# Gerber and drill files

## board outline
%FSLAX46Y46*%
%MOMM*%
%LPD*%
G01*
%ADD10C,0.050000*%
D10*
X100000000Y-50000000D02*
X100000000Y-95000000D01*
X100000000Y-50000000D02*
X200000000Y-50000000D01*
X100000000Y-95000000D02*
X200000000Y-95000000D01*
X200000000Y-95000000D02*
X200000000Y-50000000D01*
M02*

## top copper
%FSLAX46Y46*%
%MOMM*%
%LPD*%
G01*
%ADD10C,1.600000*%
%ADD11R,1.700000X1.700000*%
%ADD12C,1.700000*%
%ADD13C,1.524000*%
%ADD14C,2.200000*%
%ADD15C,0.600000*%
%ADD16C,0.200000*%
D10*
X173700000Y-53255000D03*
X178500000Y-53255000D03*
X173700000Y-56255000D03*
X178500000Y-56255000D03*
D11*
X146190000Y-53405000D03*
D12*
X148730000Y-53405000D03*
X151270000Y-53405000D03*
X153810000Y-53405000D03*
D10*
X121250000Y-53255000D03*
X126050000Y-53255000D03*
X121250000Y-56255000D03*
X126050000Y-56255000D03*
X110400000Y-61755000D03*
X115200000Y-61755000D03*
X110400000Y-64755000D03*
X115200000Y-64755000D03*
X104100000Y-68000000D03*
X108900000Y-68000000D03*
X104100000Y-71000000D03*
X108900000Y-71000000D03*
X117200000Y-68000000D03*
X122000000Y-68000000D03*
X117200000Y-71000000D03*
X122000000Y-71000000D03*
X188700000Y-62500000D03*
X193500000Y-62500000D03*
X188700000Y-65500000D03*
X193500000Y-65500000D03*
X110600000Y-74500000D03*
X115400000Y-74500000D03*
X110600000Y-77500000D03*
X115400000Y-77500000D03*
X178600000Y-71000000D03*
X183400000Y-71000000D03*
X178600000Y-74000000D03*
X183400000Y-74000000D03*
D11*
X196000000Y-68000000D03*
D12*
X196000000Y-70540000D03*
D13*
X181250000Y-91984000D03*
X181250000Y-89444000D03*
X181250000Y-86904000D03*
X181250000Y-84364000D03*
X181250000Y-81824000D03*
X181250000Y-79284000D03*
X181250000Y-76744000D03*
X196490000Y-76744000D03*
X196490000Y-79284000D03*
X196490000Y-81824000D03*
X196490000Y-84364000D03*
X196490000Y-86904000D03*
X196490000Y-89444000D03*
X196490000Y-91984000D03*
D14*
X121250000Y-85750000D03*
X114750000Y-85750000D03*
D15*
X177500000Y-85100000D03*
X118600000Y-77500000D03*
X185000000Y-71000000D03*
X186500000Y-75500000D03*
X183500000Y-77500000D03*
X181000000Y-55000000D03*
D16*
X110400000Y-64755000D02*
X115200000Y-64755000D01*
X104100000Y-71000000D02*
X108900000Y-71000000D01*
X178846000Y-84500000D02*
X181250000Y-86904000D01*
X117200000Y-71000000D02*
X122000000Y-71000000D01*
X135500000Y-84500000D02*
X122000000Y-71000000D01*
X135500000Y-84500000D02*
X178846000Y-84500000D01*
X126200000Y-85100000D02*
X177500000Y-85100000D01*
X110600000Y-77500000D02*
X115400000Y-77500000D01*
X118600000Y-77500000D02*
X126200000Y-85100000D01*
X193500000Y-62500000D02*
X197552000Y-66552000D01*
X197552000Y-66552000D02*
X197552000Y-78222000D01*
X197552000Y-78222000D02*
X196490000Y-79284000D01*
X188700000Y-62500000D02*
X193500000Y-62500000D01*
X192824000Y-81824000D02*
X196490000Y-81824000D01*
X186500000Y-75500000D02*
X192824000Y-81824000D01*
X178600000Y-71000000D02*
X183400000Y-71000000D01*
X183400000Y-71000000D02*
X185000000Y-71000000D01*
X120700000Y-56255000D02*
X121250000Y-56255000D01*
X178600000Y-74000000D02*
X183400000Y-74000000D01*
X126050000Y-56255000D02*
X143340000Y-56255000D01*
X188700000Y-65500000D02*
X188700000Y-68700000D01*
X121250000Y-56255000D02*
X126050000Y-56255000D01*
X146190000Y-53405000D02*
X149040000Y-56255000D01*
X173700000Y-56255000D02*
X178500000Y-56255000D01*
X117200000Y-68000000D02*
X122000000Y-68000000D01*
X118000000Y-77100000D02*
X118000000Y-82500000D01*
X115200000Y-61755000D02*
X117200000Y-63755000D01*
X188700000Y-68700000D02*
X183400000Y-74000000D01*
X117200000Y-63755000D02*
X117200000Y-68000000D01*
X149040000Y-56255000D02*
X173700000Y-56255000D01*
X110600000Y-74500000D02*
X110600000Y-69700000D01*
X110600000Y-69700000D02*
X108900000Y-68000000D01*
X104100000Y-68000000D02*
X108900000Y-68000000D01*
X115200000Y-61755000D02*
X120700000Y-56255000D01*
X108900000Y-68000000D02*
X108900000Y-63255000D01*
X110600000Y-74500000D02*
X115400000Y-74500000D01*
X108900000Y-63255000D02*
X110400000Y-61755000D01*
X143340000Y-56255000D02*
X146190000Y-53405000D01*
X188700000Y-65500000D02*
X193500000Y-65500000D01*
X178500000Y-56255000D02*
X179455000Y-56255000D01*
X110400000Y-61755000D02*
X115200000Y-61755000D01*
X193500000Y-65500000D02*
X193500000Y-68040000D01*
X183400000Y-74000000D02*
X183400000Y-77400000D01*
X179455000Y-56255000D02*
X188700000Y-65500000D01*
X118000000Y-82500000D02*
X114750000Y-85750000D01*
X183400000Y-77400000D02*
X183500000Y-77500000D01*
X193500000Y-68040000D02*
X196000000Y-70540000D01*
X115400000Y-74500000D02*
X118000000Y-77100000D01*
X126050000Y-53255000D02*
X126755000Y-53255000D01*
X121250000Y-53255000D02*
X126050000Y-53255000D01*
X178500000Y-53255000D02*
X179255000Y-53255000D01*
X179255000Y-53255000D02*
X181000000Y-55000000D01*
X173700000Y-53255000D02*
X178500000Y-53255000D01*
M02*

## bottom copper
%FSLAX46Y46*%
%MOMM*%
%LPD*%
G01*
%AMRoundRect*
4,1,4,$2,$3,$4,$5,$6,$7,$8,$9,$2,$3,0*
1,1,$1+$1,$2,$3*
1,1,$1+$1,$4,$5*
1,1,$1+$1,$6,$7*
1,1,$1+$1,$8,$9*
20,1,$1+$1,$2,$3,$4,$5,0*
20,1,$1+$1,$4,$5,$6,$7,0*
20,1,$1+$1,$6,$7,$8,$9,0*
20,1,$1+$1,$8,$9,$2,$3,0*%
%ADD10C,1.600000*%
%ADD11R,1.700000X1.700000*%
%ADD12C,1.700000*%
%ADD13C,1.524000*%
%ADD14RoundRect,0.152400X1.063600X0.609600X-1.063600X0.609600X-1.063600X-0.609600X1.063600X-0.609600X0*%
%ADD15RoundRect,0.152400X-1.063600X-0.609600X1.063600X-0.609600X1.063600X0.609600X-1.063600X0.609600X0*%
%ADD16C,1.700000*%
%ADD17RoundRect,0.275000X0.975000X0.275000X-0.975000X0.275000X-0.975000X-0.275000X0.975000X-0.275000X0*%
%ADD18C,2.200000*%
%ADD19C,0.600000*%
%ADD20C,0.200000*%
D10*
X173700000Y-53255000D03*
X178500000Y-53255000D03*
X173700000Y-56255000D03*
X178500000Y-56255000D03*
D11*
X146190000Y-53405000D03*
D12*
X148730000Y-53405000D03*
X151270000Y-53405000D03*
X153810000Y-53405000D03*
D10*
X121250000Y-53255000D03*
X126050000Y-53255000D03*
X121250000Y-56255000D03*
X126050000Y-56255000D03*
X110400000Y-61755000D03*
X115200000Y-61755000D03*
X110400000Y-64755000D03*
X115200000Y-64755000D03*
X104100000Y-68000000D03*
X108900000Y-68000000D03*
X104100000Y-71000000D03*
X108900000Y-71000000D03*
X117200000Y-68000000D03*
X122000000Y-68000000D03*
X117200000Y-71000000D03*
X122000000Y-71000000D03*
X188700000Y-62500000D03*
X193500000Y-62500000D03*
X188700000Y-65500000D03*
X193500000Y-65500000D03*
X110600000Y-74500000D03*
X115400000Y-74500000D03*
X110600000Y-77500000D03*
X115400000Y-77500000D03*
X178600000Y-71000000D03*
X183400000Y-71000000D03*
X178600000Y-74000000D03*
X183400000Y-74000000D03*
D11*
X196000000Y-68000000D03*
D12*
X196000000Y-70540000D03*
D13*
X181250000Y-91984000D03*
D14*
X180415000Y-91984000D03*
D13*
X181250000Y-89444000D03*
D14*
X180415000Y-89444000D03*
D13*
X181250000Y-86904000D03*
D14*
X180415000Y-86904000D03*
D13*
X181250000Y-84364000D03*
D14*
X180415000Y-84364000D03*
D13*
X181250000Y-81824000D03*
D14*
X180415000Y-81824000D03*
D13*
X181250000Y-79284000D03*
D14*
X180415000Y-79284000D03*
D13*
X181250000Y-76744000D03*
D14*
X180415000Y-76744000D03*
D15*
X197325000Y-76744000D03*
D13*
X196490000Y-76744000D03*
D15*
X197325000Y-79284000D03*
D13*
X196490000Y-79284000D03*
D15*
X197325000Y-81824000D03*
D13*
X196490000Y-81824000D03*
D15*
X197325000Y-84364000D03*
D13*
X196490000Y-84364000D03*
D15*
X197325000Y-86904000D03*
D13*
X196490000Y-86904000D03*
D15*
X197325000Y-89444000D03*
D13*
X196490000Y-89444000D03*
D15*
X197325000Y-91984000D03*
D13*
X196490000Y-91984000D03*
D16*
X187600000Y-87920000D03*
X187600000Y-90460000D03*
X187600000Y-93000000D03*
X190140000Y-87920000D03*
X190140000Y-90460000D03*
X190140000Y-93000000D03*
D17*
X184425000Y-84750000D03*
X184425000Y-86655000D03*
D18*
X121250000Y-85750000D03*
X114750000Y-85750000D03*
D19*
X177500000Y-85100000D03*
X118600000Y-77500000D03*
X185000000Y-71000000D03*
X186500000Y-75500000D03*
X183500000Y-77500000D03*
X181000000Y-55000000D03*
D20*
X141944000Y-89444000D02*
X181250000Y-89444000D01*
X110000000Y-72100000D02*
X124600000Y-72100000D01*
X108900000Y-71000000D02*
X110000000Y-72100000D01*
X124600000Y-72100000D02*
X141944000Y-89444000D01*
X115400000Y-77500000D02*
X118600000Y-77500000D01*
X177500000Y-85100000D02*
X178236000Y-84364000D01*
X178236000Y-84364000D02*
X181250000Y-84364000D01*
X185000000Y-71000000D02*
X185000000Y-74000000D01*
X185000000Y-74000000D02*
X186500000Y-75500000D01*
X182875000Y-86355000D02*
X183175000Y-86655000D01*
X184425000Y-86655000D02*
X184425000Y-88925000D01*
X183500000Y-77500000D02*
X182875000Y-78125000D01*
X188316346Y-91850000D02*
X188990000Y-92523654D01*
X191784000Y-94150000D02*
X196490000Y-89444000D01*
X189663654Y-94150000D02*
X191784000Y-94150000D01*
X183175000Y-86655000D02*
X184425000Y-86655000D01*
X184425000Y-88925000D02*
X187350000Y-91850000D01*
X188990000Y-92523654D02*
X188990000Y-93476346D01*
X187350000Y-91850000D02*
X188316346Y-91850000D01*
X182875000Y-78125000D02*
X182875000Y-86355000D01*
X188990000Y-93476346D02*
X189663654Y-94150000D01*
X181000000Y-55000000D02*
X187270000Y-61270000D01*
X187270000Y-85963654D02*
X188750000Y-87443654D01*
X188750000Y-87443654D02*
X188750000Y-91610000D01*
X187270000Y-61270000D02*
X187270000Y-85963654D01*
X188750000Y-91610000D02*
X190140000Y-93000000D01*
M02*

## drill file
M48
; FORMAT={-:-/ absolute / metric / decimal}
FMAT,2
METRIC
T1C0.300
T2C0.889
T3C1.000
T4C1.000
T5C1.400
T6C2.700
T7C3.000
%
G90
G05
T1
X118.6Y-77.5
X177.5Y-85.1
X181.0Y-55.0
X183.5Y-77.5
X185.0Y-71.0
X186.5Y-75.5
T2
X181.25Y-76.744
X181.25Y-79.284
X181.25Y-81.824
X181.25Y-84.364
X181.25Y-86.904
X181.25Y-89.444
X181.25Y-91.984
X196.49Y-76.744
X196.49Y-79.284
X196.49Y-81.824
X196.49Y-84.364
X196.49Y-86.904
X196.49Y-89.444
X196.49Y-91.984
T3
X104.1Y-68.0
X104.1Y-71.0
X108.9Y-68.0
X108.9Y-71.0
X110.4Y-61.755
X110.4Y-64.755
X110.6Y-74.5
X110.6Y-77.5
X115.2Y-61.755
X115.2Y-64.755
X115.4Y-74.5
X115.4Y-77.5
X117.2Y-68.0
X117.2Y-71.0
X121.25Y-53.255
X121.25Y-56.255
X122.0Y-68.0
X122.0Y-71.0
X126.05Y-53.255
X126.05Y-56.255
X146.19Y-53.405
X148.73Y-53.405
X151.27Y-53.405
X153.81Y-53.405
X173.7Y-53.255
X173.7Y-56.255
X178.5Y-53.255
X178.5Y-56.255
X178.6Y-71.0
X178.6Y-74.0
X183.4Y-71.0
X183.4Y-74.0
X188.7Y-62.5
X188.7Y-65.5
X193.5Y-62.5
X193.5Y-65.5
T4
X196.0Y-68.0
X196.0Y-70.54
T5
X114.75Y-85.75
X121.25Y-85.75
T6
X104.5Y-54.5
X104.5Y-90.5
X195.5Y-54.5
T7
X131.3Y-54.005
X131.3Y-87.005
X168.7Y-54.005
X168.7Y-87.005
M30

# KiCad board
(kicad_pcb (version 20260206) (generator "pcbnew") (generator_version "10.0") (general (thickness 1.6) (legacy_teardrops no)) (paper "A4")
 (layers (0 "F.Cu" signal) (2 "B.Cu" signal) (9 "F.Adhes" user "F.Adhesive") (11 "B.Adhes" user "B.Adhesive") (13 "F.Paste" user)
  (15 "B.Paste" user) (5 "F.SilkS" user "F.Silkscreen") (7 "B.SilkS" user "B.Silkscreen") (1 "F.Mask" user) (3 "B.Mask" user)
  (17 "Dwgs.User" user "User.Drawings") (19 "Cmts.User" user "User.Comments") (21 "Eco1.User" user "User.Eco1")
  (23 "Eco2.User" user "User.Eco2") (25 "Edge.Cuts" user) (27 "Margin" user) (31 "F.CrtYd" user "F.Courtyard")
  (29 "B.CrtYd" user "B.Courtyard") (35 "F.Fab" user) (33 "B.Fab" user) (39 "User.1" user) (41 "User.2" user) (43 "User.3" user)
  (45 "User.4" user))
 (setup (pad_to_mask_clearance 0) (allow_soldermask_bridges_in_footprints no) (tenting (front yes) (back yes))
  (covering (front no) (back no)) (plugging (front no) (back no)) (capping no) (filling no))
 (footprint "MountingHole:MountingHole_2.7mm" (layer "F.Cu") (at 104.5 90.5)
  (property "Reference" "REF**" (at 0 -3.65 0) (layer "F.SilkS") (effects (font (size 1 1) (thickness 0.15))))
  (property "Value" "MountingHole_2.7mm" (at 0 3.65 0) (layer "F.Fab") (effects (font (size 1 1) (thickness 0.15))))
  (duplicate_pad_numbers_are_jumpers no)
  (pad "" np_thru_hole circle (at 0 0) (size 2.7 2.7) (drill 2.7) (layers "*.Cu" "*.Mask")))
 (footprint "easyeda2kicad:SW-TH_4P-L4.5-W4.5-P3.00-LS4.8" (layer "F.Cu") (at 176.1 54.755)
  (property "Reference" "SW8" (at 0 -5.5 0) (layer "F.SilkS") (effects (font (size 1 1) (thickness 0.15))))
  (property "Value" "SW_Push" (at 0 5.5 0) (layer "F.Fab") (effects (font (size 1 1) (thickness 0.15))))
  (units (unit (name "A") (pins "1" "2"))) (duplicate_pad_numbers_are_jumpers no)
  (pad "1" thru_hole circle (at -2.4 -1.5) (size 1.6 1.6) (drill 0.999998) (layers "*.Cu" "*.Mask") (remove_unused_layers no)
   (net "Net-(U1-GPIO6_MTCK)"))
  (pad "1" thru_hole circle (at 2.4 -1.5) (size 1.6 1.6) (drill 0.999998) (layers "*.Cu" "*.Mask") (remove_unused_layers no)
   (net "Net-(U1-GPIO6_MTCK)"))
  (pad "2" thru_hole circle (at -2.4 1.5) (size 1.6 1.6) (drill 0.999998) (layers "*.Cu" "*.Mask") (remove_unused_layers no) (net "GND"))
  (pad "2" thru_hole circle (at 2.4 1.5) (size 1.6 1.6) (drill 0.999998) (layers "*.Cu" "*.Mask") (remove_unused_layers no) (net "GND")))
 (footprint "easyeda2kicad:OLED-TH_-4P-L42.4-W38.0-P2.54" (layer "F.Cu") (at 150 53.405)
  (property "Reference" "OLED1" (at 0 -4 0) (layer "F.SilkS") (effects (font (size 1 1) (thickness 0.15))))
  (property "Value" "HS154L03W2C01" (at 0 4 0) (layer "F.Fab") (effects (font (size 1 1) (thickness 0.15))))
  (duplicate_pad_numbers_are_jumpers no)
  (pad "" np_thru_hole circle (at -18.7 0.6) (size 3 3) (drill 3) (layers "*.Cu" "*.Mask"))
  (pad "" np_thru_hole circle (at -18.7 33.6) (size 3 3) (drill 3) (layers "*.Cu" "*.Mask"))
  (pad "" np_thru_hole circle (at 18.7 0.6) (size 3 3) (drill 3) (layers "*.Cu" "*.Mask"))
  (pad "" np_thru_hole circle (at 18.7 33.6) (size 3 3) (drill 3) (layers "*.Cu" "*.Mask"))
  (pad "1" thru_hole rect (at -3.81 0 270) (size 1.7 1.7) (drill 0.999998) (layers "*.Cu" "*.Mask") (remove_unused_layers no) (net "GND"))
  (pad "2" thru_hole circle (at -1.27 0 270) (size 1.7 1.7) (drill 0.999998) (layers "*.Cu" "*.Mask") (remove_unused_layers no) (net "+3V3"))
  (pad "3" thru_hole circle (at 1.27 0 270) (size 1.7 1.7) (drill 0.999998) (layers "*.Cu" "*.Mask") (remove_unused_layers no)
   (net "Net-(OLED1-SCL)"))
  (pad "4" thru_hole circle (at 3.81 0 270) (size 1.7 1.7) (drill 0.999998) (layers "*.Cu" "*.Mask") (remove_unused_layers no)
   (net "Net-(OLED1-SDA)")))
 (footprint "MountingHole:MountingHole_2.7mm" (layer "F.Cu") (at 195.5 54.5)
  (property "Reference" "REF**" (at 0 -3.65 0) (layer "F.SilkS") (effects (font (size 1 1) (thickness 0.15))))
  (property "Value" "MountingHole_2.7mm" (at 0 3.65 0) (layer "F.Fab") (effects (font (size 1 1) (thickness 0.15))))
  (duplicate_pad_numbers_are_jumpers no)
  (pad "" np_thru_hole circle (at 0 0) (size 2.7 2.7) (drill 2.7) (layers "*.Cu" "*.Mask")))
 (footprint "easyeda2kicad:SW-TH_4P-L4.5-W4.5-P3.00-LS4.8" (layer "F.Cu") (at 123.65 54.755)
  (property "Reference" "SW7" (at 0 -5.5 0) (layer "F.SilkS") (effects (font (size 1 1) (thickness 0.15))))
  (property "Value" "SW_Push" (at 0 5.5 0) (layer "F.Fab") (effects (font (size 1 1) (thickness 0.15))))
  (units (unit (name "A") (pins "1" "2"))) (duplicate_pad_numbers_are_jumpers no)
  (pad "1" thru_hole circle (at -2.4 -1.5) (size 1.6 1.6) (drill 0.999998) (layers "*.Cu" "*.Mask") (remove_unused_layers no)
   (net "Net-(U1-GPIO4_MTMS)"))
  (pad "1" thru_hole circle (at 2.4 -1.5) (size 1.6 1.6) (drill 0.999998) (layers "*.Cu" "*.Mask") (remove_unused_layers no)
   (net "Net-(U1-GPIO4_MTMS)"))
  (pad "2" thru_hole circle (at -2.4 1.5) (size 1.6 1.6) (drill 0.999998) (layers "*.Cu" "*.Mask") (remove_unused_layers no) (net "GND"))
  (pad "2" thru_hole circle (at 2.4 1.5) (size 1.6 1.6) (drill 0.999998) (layers "*.Cu" "*.Mask") (remove_unused_layers no) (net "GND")))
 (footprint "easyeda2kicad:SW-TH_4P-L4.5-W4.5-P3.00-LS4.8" (layer "F.Cu") (at 112.8 63.255)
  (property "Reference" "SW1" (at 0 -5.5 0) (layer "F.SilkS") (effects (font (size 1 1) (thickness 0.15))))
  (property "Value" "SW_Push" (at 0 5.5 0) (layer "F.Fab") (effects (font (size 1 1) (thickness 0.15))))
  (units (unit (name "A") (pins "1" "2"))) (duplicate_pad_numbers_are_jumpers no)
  (pad "1" thru_hole circle (at -2.4 -1.5) (size 1.6 1.6) (drill 0.999998) (layers "*.Cu" "*.Mask") (remove_unused_layers no) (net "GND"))
  (pad "1" thru_hole circle (at 2.4 -1.5) (size 1.6 1.6) (drill 0.999998) (layers "*.Cu" "*.Mask") (remove_unused_layers no) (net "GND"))
  (pad "2" thru_hole circle (at -2.4 1.5) (size 1.6 1.6) (drill 0.999998) (layers "*.Cu" "*.Mask") (remove_unused_layers no)
   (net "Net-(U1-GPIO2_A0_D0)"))
  (pad "2" thru_hole circle (at 2.4 1.5) (size 1.6 1.6) (drill 0.999998) (layers "*.Cu" "*.Mask") (remove_unused_layers no)
   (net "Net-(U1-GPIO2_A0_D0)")))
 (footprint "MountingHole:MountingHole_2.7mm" (layer "F.Cu") (at 104.5 54.5)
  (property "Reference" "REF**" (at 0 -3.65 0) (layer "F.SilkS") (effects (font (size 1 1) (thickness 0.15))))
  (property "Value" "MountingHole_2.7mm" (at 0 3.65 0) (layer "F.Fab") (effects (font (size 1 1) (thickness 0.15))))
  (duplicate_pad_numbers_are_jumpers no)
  (pad "" np_thru_hole circle (at 0 0) (size 2.7 2.7) (drill 2.7) (layers "*.Cu" "*.Mask")))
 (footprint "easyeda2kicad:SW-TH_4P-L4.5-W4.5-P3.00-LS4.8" (layer "F.Cu") (at 106.5 69.5)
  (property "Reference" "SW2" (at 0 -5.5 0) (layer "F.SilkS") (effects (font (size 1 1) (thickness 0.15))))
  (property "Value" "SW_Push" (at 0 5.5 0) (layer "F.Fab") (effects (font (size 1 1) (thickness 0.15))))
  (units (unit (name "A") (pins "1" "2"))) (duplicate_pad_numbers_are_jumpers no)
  (pad "1" thru_hole circle (at -2.4 -1.5) (size 1.6 1.6) (drill 0.999998) (layers "*.Cu" "*.Mask") (remove_unused_layers no) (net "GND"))
  (pad "1" thru_hole circle (at 2.4 -1.5) (size 1.6 1.6) (drill 0.999998) (layers "*.Cu" "*.Mask") (remove_unused_layers no) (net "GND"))
  (pad "2" thru_hole circle (at -2.4 1.5) (size 1.6 1.6) (drill 0.999998) (layers "*.Cu" "*.Mask") (remove_unused_layers no)
   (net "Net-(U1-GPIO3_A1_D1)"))
  (pad "2" thru_hole circle (at 2.4 1.5) (size 1.6 1.6) (drill 0.999998) (layers "*.Cu" "*.Mask") (remove_unused_layers no)
   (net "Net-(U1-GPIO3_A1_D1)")))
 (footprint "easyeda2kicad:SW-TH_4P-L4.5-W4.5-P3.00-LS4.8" (layer "F.Cu") (at 119.6 69.5)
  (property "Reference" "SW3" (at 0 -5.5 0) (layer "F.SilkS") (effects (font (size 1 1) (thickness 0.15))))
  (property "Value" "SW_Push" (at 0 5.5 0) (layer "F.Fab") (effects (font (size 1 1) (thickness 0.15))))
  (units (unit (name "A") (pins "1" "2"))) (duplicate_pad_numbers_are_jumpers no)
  (pad "1" thru_hole circle (at -2.4 -1.5) (size 1.6 1.6) (drill 0.999998) (layers "*.Cu" "*.Mask") (remove_unused_layers no) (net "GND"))
  (pad "1" thru_hole circle (at 2.4 -1.5) (size 1.6 1.6) (drill 0.999998) (layers "*.Cu" "*.Mask") (remove_unused_layers no) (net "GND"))
  (pad "2" thru_hole circle (at -2.4 1.5) (size 1.6 1.6) (drill 0.999998) (layers "*.Cu" "*.Mask") (remove_unused_layers no)
   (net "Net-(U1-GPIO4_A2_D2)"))
  (pad "2" thru_hole circle (at 2.4 1.5) (size 1.6 1.6) (drill 0.999998) (layers "*.Cu" "*.Mask") (remove_unused_layers no)
   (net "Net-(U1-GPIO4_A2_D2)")))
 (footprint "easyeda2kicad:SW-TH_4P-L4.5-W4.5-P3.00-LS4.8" (layer "F.Cu") (at 191.1 64)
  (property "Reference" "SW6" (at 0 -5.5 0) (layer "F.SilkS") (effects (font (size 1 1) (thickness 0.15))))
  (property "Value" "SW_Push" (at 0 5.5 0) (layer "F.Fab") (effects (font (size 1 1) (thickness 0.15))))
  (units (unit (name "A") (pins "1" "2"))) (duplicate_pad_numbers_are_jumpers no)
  (pad "1" thru_hole circle (at -2.4 -1.5) (size 1.6 1.6) (drill 0.999998) (layers "*.Cu" "*.Mask") (remove_unused_layers no)
   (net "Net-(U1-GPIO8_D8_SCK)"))
  (pad "1" thru_hole circle (at 2.4 -1.5) (size 1.6 1.6) (drill 0.999998) (layers "*.Cu" "*.Mask") (remove_unused_layers no)
   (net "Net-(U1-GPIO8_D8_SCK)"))
  (pad "2" thru_hole circle (at -2.4 1.5) (size 1.6 1.6) (drill 0.999998) (layers "*.Cu" "*.Mask") (remove_unused_layers no) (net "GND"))
  (pad "2" thru_hole circle (at 2.4 1.5) (size 1.6 1.6) (drill 0.999998) (layers "*.Cu" "*.Mask") (remove_unused_layers no) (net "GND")))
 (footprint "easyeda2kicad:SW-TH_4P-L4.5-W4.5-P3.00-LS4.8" (layer "F.Cu") (at 113 76)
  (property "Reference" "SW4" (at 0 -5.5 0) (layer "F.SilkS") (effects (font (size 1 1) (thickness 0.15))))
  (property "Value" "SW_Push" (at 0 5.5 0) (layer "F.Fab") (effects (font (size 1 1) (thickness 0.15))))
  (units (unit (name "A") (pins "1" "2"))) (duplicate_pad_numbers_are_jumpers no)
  (pad "1" thru_hole circle (at -2.4 -1.5) (size 1.6 1.6) (drill 0.999998) (layers "*.Cu" "*.Mask") (remove_unused_layers no) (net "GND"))
  (pad "1" thru_hole circle (at 2.4 -1.5) (size 1.6 1.6) (drill 0.999998) (layers "*.Cu" "*.Mask") (remove_unused_layers no) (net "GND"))
  (pad "2" thru_hole circle (at -2.4 1.5) (size 1.6 1.6) (drill 0.999998) (layers "*.Cu" "*.Mask") (remove_unused_layers no)
   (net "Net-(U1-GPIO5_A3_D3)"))
  (pad "2" thru_hole circle (at 2.4 1.5) (size 1.6 1.6) (drill 0.999998) (layers "*.Cu" "*.Mask") (remove_unused_layers no)
   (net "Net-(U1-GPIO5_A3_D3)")))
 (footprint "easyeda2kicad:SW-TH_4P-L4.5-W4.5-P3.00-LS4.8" (layer "F.Cu") (at 181 72.5)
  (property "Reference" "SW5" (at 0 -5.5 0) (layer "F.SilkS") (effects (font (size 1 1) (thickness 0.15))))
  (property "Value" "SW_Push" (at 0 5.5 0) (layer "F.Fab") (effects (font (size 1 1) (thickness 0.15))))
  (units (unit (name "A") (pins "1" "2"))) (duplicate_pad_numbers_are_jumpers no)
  (pad "1" thru_hole circle (at -2.4 -1.5) (size 1.6 1.6) (drill 0.999998) (layers "*.Cu" "*.Mask") (remove_unused_layers no)
   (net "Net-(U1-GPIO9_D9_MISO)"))
  (pad "1" thru_hole circle (at 2.4 -1.5) (size 1.6 1.6) (drill 0.999998) (layers "*.Cu" "*.Mask") (remove_unused_layers no)
   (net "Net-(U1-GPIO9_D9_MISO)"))
  (pad "2" thru_hole circle (at -2.4 1.5) (size 1.6 1.6) (drill 0.999998) (layers "*.Cu" "*.Mask") (remove_unused_layers no) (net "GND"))
  (pad "2" thru_hole circle (at 2.4 1.5) (size 1.6 1.6) (drill 0.999998) (layers "*.Cu" "*.Mask") (remove_unused_layers no) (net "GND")))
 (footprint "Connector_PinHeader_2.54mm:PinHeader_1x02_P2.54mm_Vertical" (layer "B.Cu") (at 196 68 180)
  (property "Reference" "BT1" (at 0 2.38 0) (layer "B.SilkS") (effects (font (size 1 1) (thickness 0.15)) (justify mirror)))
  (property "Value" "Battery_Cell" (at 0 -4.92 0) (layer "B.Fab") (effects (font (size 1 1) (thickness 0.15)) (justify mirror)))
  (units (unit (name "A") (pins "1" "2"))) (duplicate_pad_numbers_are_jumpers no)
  (pad "1" thru_hole rect (at 0 0 180) (size 1.7 1.7) (drill 1) (layers "*.Cu" "*.Mask") (remove_unused_layers no) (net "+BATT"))
  (pad "2" thru_hole circle (at 0 -2.54 180) (size 1.7 1.7) (drill 1) (layers "*.Cu" "*.Mask") (remove_unused_layers no) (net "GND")))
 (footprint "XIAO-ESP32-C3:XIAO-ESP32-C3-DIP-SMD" (layer "B.Cu") (at 188.87 84.364 -90)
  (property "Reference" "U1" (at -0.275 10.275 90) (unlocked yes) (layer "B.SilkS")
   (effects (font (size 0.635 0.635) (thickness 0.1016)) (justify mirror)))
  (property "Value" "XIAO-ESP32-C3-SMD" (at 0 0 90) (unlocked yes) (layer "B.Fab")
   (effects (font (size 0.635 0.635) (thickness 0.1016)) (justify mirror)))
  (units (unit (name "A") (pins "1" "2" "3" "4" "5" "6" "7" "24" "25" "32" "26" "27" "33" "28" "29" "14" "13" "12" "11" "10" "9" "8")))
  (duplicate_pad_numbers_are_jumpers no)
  (pad "1" thru_hole circle (at 7.62 7.62 180) (size 1.524 1.524) (drill 0.889) (layers "*.Cu" "*.Mask") (remove_unused_layers no)
   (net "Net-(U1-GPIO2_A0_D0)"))
  (pad "1" smd roundrect (at 7.62 8.455 180) (size 2.432 1.524) (layers "B.Cu" "B.Mask") (roundrect_rratio 0.1) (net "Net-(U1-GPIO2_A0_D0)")
   (thermal_bridge_angle 45))
  (pad "2" thru_hole circle (at 5.08 7.62 180) (size 1.524 1.524) (drill 0.889) (layers "*.Cu" "*.Mask") (remove_unused_layers no)
   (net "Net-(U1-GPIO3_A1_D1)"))
  (pad "2" smd roundrect (at 5.08 8.455 180) (size 2.432 1.524) (layers "B.Cu" "B.Mask") (roundrect_rratio 0.1) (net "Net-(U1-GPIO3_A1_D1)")
   (thermal_bridge_angle 45))
  (pad "3" thru_hole circle (at 2.54 7.62 180) (size 1.524 1.524) (drill 0.889) (layers "*.Cu" "*.Mask") (remove_unused_layers no)
   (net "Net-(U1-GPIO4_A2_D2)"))
  (pad "3" smd roundrect (at 2.54 8.455 180) (size 2.432 1.524) (layers "B.Cu" "B.Mask") (roundrect_rratio 0.1) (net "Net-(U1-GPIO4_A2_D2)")
   (thermal_bridge_angle 45))
  (pad "4" thru_hole circle (at 0 7.62 180) (size 1.524 1.524) (drill 0.889) (layers "*.Cu" "*.Mask") (remove_unused_layers no)
   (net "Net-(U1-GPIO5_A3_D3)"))
  (pad "4" smd roundrect (at 0 8.455 180) (size 2.432 1.524) (layers "B.Cu" "B.Mask") (roundrect_rratio 0.1) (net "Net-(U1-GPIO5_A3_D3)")
   (thermal_bridge_angle 45))
  (pad "5" thru_hole circle (at -2.54 7.62 180) (size 1.524 1.524) (drill 0.889) (layers "*.Cu" "*.Mask") (remove_unused_layers no)
   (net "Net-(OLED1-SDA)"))
  (pad "5" smd roundrect (at -2.54 8.455 180) (size 2.432 1.524) (layers "B.Cu" "B.Mask") (roundrect_rratio 0.1) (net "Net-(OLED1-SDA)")
   (thermal_bridge_angle 45))
  (pad "6" thru_hole circle (at -5.08 7.62 180) (size 1.524 1.524) (drill 0.889) (layers "*.Cu" "*.Mask") (remove_unused_layers no)
   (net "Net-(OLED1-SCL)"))
  (pad "6" smd roundrect (at -5.08 8.455 180) (size 2.432 1.524) (layers "B.Cu" "B.Mask") (roundrect_rratio 0.1) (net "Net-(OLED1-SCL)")
   (thermal_bridge_angle 45))
  (pad "7" thru_hole circle (at -7.62 7.62 180) (size 1.524 1.524) (drill 0.889) (layers "*.Cu" "*.Mask") (remove_unused_layers no)
   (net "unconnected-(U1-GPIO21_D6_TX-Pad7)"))
  (pad "7" smd roundrect (at -7.62 8.455 180) (size 2.432 1.524) (layers "B.Cu" "B.Mask") (roundrect_rratio 0.1)
   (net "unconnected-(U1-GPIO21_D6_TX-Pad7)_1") (thermal_bridge_angle 45))
  (pad "8" smd roundrect (at -7.62 -8.455) (size 2.432 1.524) (layers "B.Cu" "B.Mask") (roundrect_rratio 0.1)
   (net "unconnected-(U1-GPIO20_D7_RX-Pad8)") (thermal_bridge_angle 45))
  (pad "8" thru_hole circle (at -7.62 -7.62) (size 1.524 1.524) (drill 0.889) (layers "*.Cu" "*.Mask") (remove_unused_layers no)
   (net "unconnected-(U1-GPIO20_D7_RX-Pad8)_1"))
  (pad "9" smd roundrect (at -5.08 -8.455) (size 2.432 1.524) (layers "B.Cu" "B.Mask") (roundrect_rratio 0.1) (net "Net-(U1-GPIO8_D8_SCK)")
   (thermal_bridge_angle 45))
  (pad "9" thru_hole circle (at -5.08 -7.62) (size 1.524 1.524) (drill 0.889) (layers "*.Cu" "*.Mask") (remove_unused_layers no)
   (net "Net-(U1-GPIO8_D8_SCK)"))
  (pad "10" smd roundrect (at -2.54 -8.455) (size 2.432 1.524) (layers "B.Cu" "B.Mask") (roundrect_rratio 0.1)
   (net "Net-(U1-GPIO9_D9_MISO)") (thermal_bridge_angle 45))
  (pad "10" thru_hole circle (at -2.54 -7.62) (size 1.524 1.524) (drill 0.889) (layers "*.Cu" "*.Mask") (remove_unused_layers no)
   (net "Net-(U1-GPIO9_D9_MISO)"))
  (pad "11" smd roundrect (at 0 -8.455) (size 2.432 1.524) (layers "B.Cu" "B.Mask") (roundrect_rratio 0.1) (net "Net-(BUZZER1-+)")
   (thermal_bridge_angle 45))
  (pad "11" thru_hole circle (at 0 -7.62) (size 1.524 1.524) (drill 0.889) (layers "*.Cu" "*.Mask") (remove_unused_layers no)
   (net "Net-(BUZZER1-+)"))
  (pad "12" smd roundrect (at 2.54 -8.455) (size 2.432 1.524) (layers "B.Cu" "B.Mask") (roundrect_rratio 0.1) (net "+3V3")
   (thermal_bridge_angle 45))
  (pad "12" thru_hole circle (at 2.54 -7.62) (size 1.524 1.524) (drill 0.889) (layers "*.Cu" "*.Mask") (remove_unused_layers no)
   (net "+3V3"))
  (pad "13" smd roundrect (at 5.08 -8.455) (size 2.432 1.524) (layers "B.Cu" "B.Mask") (roundrect_rratio 0.1) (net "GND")
   (thermal_bridge_angle 45))
  (pad "13" thru_hole circle (at 5.08 -7.62) (size 1.524 1.524) (drill 0.889) (layers "*.Cu" "*.Mask") (remove_unused_layers no) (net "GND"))
  (pad "14" smd roundrect (at 7.62 -8.455) (size 2.432 1.524) (layers "B.Cu" "B.Mask") (roundrect_rratio 0.1) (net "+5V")
   (thermal_bridge_angle 45))
  (pad "14" thru_hole circle (at 7.62 -7.62) (size 1.524 1.524) (drill 0.889) (layers "*.Cu" "*.Mask") (remove_unused_layers no) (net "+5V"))
  (pad "24" smd circle (at 3.556 1.27) (size 1.7 1.7) (layers "B.Cu" "B.Mask" "B.Paste") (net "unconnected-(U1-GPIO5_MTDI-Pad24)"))
  (pad "25" smd circle (at 6.096 1.27) (size 1.7 1.7) (layers "B.Cu" "B.Mask" "B.Paste") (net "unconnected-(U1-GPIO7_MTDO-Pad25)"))
  (pad "26" smd circle (at 8.636 1.27) (size 1.7 1.7) (layers "B.Cu" "B.Mask" "B.Paste") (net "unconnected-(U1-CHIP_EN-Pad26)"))
  (pad "27" smd circle (at 3.556 -1.27) (size 1.7 1.7) (layers "B.Cu" "B.Mask" "B.Paste") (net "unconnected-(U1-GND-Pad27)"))
  (pad "28" smd circle (at 6.096 -1.27) (size 1.7 1.7) (layers "B.Cu" "B.Mask" "B.Paste") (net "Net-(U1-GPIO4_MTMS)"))
  (pad "29" smd circle (at 8.636 -1.27) (size 1.7 1.7) (layers "B.Cu" "B.Mask" "B.Paste") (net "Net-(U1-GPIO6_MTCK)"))
  (pad "32" smd roundrect (at 0.386 4.445 180) (size 2.5 1.1) (layers "B.Cu" "B.Mask" "B.Paste") (roundrect_rratio 0.25) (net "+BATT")
   (thermal_bridge_angle 45))
  (pad "33" smd roundrect (at 2.291 4.445 180) (size 2.5 1.1) (layers "B.Cu" "B.Mask" "B.Paste") (roundrect_rratio 0.25) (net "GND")
   (thermal_bridge_angle 45)))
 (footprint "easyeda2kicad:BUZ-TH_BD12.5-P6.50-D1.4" (layer "B.Cu") (at 118 85.75 180)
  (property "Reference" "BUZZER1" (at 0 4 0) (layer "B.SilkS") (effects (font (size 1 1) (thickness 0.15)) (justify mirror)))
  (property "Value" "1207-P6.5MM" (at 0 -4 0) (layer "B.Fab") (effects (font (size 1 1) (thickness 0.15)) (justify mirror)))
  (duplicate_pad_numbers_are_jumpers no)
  (pad "1" thru_hole circle (at -3.25 0 180) (size 2.2 2.2) (drill 1.399998) (layers "*.Cu" "*.Mask") (remove_unused_layers no)
   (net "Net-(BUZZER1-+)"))
  (pad "2" thru_hole circle (at 3.25 0 180) (size 2.2 2.2) (drill 1.399998) (layers "*.Cu" "*.Mask") (remove_unused_layers no) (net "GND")))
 (gr_line (start 100 50) (end 100 95) (stroke (width 0.05) (type default)) (layer "Edge.Cuts"))
 (gr_line (start 100 50) (end 200 50) (stroke (width 0.05) (type default)) (layer "Edge.Cuts"))
 (gr_line (start 100 95) (end 200 95) (stroke (width 0.05) (type default)) (layer "Edge.Cuts"))
 (gr_line (start 200 95) (end 200 50) (stroke (width 0.05) (type default)) (layer "Edge.Cuts"))
 (segment (start 110.4 64.755) (end 115.2 64.755) (width 0.2) (layer "F.Cu") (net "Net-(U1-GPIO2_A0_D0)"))
 (segment (start 104.1 71) (end 108.9 71) (width 0.2) (layer "F.Cu") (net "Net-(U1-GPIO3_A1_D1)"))
 (segment (start 141.944 89.444) (end 181.25 89.444) (width 0.2) (layer "B.Cu") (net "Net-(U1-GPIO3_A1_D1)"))
 (segment (start 110 72.1) (end 124.6 72.1) (width 0.2) (layer "B.Cu") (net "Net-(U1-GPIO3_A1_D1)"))
 (segment (start 108.9 71) (end 110 72.1) (width 0.2) (layer "B.Cu") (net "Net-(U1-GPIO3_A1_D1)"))
 (segment (start 124.6 72.1) (end 141.944 89.444) (width 0.2) (layer "B.Cu") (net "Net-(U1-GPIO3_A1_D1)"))
 (segment (start 178.846 84.5) (end 181.25 86.904) (width 0.2) (layer "F.Cu") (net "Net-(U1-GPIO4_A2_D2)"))
 (segment (start 117.2 71) (end 122 71) (width 0.2) (layer "F.Cu") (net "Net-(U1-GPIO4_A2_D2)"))
 (segment (start 135.5 84.5) (end 122 71) (width 0.2) (layer "F.Cu") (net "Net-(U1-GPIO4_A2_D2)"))
 (segment (start 135.5 84.5) (end 178.846 84.5) (width 0.2) (layer "F.Cu") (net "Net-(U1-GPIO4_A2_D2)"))
 (segment (start 126.2 85.1) (end 177.5 85.1) (width 0.2) (layer "F.Cu") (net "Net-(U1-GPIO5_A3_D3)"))
 (segment (start 110.6 77.5) (end 115.4 77.5) (width 0.2) (layer "F.Cu") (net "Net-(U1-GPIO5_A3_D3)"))
 (segment (start 118.6 77.5) (end 126.2 85.1) (width 0.2) (layer "F.Cu") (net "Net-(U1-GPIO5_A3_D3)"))
 (via (at 177.5 85.1) (size 0.6) (drill 0.3) (layers "F.Cu" "B.Cu") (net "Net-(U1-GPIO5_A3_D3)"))
 (via (at 118.6 77.5) (size 0.6) (drill 0.3) (layers "F.Cu" "B.Cu") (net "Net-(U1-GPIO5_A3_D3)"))
 (segment (start 115.4 77.5) (end 118.6 77.5) (width 0.2) (layer "B.Cu") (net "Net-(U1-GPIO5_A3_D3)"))
 (segment (start 177.5 85.1) (end 178.236 84.364) (width 0.2) (layer "B.Cu") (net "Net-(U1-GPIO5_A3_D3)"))
 (segment (start 178.236 84.364) (end 181.25 84.364) (width 0.2) (layer "B.Cu") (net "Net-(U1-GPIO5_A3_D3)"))
 (segment (start 193.5 62.5) (end 197.552 66.552) (width 0.2) (layer "F.Cu") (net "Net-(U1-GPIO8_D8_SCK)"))
 (segment (start 197.552 66.552) (end 197.552 78.222) (width 0.2) (layer "F.Cu") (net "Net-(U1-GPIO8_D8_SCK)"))
 (segment (start 197.552 78.222) (end 196.49 79.284) (width 0.2) (layer "F.Cu") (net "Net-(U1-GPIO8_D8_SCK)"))
 (segment (start 188.7 62.5) (end 193.5 62.5) (width 0.2) (layer "F.Cu") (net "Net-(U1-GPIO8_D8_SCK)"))
 (segment (start 192.824 81.824) (end 196.49 81.824) (width 0.2) (layer "F.Cu") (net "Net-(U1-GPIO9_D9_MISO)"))
 (segment (start 186.5 75.5) (end 192.824 81.824) (width 0.2) (layer "F.Cu") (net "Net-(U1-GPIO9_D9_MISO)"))
 (segment (start 178.6 71) (end 183.4 71) (width 0.2) (layer "F.Cu") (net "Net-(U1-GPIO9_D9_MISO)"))
 (segment (start 183.4 71) (end 185 71) (width 0.2) (layer "F.Cu") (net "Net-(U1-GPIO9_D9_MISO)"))
 (via (at 185 71) (size 0.6) (drill 0.3) (layers "F.Cu" "B.Cu") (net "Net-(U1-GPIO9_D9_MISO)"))
 (via (at 186.5 75.5) (size 0.6) (drill 0.3) (layers "F.Cu" "B.Cu") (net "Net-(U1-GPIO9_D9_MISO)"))
 (segment (start 185 71) (end 185 74) (width 0.2) (layer "B.Cu") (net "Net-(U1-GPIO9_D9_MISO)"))
 (segment (start 185 74) (end 186.5 75.5) (width 0.2) (layer "B.Cu") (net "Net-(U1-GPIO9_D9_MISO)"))
 (segment (start 120.7 56.255) (end 121.25 56.255) (width 0.2) (layer "F.Cu") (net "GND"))
 (segment (start 178.6 74) (end 183.4 74) (width 0.2) (layer "F.Cu") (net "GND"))
 (segment (start 126.05 56.255) (end 143.34 56.255) (width 0.2) (layer "F.Cu") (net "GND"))
 (segment (start 188.7 65.5) (end 188.7 68.7) (width 0.2) (layer "F.Cu") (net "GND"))
 (segment (start 121.25 56.255) (end 126.05 56.255) (width 0.2) (layer "F.Cu") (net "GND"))
 (segment (start 146.19 53.405) (end 149.04 56.255) (width 0.2) (layer "F.Cu") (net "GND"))
 (segment (start 173.7 56.255) (end 178.5 56.255) (width 0.2) (layer "F.Cu") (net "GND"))
 (segment (start 117.2 68) (end 122 68) (width 0.2) (layer "F.Cu") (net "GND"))
 (segment (start 118 77.1) (end 118 82.5) (width 0.2) (layer "F.Cu") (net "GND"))
 (segment (start 115.2 61.755) (end 117.2 63.755) (width 0.2) (layer "F.Cu") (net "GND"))
 (segment (start 188.7 68.7) (end 183.4 74) (width 0.2) (layer "F.Cu") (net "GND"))
 (segment (start 117.2 63.755) (end 117.2 68) (width 0.2) (layer "F.Cu") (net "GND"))
 (segment (start 149.04 56.255) (end 173.7 56.255) (width 0.2) (layer "F.Cu") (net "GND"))
 (segment (start 110.6 74.5) (end 110.6 69.7) (width 0.2) (layer "F.Cu") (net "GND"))
 (segment (start 110.6 69.7) (end 108.9 68) (width 0.2) (layer "F.Cu") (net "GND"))
 (segment (start 104.1 68) (end 108.9 68) (width 0.2) (layer "F.Cu") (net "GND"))
 (segment (start 115.2 61.755) (end 120.7 56.255) (width 0.2) (layer "F.Cu") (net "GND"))
 (segment (start 108.9 68) (end 108.9 63.255) (width 0.2) (layer "F.Cu") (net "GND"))
 (segment (start 110.6 74.5) (end 115.4 74.5) (width 0.2) (layer "F.Cu") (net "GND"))
 (segment (start 108.9 63.255) (end 110.4 61.755) (width 0.2) (layer "F.Cu") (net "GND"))
 (segment (start 143.34 56.255) (end 146.19 53.405) (width 0.2) (layer "F.Cu") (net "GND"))
 (segment (start 188.7 65.5) (end 193.5 65.5) (width 0.2) (layer "F.Cu") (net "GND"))
 (segment (start 178.5 56.255) (end 179.455 56.255) (width 0.2) (layer "F.Cu") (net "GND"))
 (segment (start 110.4 61.755) (end 115.2 61.755) (width 0.2) (layer "F.Cu") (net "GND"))
 (segment (start 193.5 65.5) (end 193.5 68.04) (width 0.2) (layer "F.Cu") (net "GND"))
 (segment (start 183.4 74) (end 183.4 77.4) (width 0.2) (layer "F.Cu") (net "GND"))
 (segment (start 179.455 56.255) (end 188.7 65.5) (width 0.2) (layer "F.Cu") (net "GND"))
 (segment (start 118 82.5) (end 114.75 85.75) (width 0.2) (layer "F.Cu") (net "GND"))
 (segment (start 183.4 77.4) (end 183.5 77.5) (width 0.2) (layer "F.Cu") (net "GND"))
 (segment (start 193.5 68.04) (end 196 70.54) (width 0.2) (layer "F.Cu") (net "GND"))
 (segment (start 115.4 74.5) (end 118 77.1) (width 0.2) (layer "F.Cu") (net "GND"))
 (via (at 183.5 77.5) (size 0.6) (drill 0.3) (layers "F.Cu" "B.Cu") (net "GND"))
 (segment (start 182.875 86.355) (end 183.175 86.655) (width 0.2) (layer "B.Cu") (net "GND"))
 (segment (start 184.425 86.655) (end 184.425 88.925) (width 0.2) (layer "B.Cu") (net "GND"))
 (segment (start 183.5 77.5) (end 182.875 78.125) (width 0.2) (layer "B.Cu") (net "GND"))
 (segment (start 188.316346 91.85) (end 188.99 92.523654) (width 0.2) (layer "B.Cu") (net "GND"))
 (segment (start 191.784 94.15) (end 196.49 89.444) (width 0.2) (layer "B.Cu") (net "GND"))
 (segment (start 189.663654 94.15) (end 191.784 94.15) (width 0.2) (layer "B.Cu") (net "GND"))
 (segment (start 183.175 86.655) (end 184.425 86.655) (width 0.2) (layer "B.Cu") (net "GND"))
 (segment (start 184.425 88.925) (end 187.35 91.85) (width 0.2) (layer "B.Cu") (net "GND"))
 (segment (start 188.99 92.523654) (end 188.99 93.476346) (width 0.2) (layer "B.Cu") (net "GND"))
 (segment (start 187.35 91.85) (end 188.316346 91.85) (width 0.2) (layer "B.Cu") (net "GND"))
 (segment (start 182.875 78.125) (end 182.875 86.355) (width 0.2) (layer "B.Cu") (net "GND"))
 (segment (start 188.99 93.476346) (end 189.663654 94.15) (width 0.2) (layer "B.Cu") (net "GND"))
 (segment (start 126.05 53.255) (end 126.755 53.255) (width 0.2) (layer "F.Cu") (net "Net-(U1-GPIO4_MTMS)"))
 (segment (start 121.25 53.255) (end 126.05 53.255) (width 0.2) (layer "F.Cu") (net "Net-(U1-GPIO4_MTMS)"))
 (segment (start 178.5 53.255) (end 179.255 53.255) (width 0.2) (layer "F.Cu") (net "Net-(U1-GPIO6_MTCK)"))
 (segment (start 179.255 53.255) (end 181 55) (width 0.2) (layer "F.Cu") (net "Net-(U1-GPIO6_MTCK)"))
 (segment (start 173.7 53.255) (end 178.5 53.255) (width 0.2) (layer "F.Cu") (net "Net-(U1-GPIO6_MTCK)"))
 (via (at 181 55) (size 0.6) (drill 0.3) (layers "F.Cu" "B.Cu") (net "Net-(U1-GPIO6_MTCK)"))
 (segment (start 181 55) (end 187.27 61.27) (width 0.2) (layer "B.Cu") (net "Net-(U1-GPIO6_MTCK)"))
 (segment (start 187.27 85.963654) (end 188.75 87.443654) (width 0.2) (layer "B.Cu") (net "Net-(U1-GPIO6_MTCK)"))
 (segment (start 188.75 87.443654) (end 188.75 91.61) (width 0.2) (layer "B.Cu") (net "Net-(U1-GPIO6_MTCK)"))
 (segment (start 187.27 61.27) (end 187.27 85.963654) (width 0.2) (layer "B.Cu") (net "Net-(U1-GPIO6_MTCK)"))
 (segment (start 188.75 91.61) (end 190.14 93) (width 0.2) (layer "B.Cu") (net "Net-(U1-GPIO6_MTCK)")))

